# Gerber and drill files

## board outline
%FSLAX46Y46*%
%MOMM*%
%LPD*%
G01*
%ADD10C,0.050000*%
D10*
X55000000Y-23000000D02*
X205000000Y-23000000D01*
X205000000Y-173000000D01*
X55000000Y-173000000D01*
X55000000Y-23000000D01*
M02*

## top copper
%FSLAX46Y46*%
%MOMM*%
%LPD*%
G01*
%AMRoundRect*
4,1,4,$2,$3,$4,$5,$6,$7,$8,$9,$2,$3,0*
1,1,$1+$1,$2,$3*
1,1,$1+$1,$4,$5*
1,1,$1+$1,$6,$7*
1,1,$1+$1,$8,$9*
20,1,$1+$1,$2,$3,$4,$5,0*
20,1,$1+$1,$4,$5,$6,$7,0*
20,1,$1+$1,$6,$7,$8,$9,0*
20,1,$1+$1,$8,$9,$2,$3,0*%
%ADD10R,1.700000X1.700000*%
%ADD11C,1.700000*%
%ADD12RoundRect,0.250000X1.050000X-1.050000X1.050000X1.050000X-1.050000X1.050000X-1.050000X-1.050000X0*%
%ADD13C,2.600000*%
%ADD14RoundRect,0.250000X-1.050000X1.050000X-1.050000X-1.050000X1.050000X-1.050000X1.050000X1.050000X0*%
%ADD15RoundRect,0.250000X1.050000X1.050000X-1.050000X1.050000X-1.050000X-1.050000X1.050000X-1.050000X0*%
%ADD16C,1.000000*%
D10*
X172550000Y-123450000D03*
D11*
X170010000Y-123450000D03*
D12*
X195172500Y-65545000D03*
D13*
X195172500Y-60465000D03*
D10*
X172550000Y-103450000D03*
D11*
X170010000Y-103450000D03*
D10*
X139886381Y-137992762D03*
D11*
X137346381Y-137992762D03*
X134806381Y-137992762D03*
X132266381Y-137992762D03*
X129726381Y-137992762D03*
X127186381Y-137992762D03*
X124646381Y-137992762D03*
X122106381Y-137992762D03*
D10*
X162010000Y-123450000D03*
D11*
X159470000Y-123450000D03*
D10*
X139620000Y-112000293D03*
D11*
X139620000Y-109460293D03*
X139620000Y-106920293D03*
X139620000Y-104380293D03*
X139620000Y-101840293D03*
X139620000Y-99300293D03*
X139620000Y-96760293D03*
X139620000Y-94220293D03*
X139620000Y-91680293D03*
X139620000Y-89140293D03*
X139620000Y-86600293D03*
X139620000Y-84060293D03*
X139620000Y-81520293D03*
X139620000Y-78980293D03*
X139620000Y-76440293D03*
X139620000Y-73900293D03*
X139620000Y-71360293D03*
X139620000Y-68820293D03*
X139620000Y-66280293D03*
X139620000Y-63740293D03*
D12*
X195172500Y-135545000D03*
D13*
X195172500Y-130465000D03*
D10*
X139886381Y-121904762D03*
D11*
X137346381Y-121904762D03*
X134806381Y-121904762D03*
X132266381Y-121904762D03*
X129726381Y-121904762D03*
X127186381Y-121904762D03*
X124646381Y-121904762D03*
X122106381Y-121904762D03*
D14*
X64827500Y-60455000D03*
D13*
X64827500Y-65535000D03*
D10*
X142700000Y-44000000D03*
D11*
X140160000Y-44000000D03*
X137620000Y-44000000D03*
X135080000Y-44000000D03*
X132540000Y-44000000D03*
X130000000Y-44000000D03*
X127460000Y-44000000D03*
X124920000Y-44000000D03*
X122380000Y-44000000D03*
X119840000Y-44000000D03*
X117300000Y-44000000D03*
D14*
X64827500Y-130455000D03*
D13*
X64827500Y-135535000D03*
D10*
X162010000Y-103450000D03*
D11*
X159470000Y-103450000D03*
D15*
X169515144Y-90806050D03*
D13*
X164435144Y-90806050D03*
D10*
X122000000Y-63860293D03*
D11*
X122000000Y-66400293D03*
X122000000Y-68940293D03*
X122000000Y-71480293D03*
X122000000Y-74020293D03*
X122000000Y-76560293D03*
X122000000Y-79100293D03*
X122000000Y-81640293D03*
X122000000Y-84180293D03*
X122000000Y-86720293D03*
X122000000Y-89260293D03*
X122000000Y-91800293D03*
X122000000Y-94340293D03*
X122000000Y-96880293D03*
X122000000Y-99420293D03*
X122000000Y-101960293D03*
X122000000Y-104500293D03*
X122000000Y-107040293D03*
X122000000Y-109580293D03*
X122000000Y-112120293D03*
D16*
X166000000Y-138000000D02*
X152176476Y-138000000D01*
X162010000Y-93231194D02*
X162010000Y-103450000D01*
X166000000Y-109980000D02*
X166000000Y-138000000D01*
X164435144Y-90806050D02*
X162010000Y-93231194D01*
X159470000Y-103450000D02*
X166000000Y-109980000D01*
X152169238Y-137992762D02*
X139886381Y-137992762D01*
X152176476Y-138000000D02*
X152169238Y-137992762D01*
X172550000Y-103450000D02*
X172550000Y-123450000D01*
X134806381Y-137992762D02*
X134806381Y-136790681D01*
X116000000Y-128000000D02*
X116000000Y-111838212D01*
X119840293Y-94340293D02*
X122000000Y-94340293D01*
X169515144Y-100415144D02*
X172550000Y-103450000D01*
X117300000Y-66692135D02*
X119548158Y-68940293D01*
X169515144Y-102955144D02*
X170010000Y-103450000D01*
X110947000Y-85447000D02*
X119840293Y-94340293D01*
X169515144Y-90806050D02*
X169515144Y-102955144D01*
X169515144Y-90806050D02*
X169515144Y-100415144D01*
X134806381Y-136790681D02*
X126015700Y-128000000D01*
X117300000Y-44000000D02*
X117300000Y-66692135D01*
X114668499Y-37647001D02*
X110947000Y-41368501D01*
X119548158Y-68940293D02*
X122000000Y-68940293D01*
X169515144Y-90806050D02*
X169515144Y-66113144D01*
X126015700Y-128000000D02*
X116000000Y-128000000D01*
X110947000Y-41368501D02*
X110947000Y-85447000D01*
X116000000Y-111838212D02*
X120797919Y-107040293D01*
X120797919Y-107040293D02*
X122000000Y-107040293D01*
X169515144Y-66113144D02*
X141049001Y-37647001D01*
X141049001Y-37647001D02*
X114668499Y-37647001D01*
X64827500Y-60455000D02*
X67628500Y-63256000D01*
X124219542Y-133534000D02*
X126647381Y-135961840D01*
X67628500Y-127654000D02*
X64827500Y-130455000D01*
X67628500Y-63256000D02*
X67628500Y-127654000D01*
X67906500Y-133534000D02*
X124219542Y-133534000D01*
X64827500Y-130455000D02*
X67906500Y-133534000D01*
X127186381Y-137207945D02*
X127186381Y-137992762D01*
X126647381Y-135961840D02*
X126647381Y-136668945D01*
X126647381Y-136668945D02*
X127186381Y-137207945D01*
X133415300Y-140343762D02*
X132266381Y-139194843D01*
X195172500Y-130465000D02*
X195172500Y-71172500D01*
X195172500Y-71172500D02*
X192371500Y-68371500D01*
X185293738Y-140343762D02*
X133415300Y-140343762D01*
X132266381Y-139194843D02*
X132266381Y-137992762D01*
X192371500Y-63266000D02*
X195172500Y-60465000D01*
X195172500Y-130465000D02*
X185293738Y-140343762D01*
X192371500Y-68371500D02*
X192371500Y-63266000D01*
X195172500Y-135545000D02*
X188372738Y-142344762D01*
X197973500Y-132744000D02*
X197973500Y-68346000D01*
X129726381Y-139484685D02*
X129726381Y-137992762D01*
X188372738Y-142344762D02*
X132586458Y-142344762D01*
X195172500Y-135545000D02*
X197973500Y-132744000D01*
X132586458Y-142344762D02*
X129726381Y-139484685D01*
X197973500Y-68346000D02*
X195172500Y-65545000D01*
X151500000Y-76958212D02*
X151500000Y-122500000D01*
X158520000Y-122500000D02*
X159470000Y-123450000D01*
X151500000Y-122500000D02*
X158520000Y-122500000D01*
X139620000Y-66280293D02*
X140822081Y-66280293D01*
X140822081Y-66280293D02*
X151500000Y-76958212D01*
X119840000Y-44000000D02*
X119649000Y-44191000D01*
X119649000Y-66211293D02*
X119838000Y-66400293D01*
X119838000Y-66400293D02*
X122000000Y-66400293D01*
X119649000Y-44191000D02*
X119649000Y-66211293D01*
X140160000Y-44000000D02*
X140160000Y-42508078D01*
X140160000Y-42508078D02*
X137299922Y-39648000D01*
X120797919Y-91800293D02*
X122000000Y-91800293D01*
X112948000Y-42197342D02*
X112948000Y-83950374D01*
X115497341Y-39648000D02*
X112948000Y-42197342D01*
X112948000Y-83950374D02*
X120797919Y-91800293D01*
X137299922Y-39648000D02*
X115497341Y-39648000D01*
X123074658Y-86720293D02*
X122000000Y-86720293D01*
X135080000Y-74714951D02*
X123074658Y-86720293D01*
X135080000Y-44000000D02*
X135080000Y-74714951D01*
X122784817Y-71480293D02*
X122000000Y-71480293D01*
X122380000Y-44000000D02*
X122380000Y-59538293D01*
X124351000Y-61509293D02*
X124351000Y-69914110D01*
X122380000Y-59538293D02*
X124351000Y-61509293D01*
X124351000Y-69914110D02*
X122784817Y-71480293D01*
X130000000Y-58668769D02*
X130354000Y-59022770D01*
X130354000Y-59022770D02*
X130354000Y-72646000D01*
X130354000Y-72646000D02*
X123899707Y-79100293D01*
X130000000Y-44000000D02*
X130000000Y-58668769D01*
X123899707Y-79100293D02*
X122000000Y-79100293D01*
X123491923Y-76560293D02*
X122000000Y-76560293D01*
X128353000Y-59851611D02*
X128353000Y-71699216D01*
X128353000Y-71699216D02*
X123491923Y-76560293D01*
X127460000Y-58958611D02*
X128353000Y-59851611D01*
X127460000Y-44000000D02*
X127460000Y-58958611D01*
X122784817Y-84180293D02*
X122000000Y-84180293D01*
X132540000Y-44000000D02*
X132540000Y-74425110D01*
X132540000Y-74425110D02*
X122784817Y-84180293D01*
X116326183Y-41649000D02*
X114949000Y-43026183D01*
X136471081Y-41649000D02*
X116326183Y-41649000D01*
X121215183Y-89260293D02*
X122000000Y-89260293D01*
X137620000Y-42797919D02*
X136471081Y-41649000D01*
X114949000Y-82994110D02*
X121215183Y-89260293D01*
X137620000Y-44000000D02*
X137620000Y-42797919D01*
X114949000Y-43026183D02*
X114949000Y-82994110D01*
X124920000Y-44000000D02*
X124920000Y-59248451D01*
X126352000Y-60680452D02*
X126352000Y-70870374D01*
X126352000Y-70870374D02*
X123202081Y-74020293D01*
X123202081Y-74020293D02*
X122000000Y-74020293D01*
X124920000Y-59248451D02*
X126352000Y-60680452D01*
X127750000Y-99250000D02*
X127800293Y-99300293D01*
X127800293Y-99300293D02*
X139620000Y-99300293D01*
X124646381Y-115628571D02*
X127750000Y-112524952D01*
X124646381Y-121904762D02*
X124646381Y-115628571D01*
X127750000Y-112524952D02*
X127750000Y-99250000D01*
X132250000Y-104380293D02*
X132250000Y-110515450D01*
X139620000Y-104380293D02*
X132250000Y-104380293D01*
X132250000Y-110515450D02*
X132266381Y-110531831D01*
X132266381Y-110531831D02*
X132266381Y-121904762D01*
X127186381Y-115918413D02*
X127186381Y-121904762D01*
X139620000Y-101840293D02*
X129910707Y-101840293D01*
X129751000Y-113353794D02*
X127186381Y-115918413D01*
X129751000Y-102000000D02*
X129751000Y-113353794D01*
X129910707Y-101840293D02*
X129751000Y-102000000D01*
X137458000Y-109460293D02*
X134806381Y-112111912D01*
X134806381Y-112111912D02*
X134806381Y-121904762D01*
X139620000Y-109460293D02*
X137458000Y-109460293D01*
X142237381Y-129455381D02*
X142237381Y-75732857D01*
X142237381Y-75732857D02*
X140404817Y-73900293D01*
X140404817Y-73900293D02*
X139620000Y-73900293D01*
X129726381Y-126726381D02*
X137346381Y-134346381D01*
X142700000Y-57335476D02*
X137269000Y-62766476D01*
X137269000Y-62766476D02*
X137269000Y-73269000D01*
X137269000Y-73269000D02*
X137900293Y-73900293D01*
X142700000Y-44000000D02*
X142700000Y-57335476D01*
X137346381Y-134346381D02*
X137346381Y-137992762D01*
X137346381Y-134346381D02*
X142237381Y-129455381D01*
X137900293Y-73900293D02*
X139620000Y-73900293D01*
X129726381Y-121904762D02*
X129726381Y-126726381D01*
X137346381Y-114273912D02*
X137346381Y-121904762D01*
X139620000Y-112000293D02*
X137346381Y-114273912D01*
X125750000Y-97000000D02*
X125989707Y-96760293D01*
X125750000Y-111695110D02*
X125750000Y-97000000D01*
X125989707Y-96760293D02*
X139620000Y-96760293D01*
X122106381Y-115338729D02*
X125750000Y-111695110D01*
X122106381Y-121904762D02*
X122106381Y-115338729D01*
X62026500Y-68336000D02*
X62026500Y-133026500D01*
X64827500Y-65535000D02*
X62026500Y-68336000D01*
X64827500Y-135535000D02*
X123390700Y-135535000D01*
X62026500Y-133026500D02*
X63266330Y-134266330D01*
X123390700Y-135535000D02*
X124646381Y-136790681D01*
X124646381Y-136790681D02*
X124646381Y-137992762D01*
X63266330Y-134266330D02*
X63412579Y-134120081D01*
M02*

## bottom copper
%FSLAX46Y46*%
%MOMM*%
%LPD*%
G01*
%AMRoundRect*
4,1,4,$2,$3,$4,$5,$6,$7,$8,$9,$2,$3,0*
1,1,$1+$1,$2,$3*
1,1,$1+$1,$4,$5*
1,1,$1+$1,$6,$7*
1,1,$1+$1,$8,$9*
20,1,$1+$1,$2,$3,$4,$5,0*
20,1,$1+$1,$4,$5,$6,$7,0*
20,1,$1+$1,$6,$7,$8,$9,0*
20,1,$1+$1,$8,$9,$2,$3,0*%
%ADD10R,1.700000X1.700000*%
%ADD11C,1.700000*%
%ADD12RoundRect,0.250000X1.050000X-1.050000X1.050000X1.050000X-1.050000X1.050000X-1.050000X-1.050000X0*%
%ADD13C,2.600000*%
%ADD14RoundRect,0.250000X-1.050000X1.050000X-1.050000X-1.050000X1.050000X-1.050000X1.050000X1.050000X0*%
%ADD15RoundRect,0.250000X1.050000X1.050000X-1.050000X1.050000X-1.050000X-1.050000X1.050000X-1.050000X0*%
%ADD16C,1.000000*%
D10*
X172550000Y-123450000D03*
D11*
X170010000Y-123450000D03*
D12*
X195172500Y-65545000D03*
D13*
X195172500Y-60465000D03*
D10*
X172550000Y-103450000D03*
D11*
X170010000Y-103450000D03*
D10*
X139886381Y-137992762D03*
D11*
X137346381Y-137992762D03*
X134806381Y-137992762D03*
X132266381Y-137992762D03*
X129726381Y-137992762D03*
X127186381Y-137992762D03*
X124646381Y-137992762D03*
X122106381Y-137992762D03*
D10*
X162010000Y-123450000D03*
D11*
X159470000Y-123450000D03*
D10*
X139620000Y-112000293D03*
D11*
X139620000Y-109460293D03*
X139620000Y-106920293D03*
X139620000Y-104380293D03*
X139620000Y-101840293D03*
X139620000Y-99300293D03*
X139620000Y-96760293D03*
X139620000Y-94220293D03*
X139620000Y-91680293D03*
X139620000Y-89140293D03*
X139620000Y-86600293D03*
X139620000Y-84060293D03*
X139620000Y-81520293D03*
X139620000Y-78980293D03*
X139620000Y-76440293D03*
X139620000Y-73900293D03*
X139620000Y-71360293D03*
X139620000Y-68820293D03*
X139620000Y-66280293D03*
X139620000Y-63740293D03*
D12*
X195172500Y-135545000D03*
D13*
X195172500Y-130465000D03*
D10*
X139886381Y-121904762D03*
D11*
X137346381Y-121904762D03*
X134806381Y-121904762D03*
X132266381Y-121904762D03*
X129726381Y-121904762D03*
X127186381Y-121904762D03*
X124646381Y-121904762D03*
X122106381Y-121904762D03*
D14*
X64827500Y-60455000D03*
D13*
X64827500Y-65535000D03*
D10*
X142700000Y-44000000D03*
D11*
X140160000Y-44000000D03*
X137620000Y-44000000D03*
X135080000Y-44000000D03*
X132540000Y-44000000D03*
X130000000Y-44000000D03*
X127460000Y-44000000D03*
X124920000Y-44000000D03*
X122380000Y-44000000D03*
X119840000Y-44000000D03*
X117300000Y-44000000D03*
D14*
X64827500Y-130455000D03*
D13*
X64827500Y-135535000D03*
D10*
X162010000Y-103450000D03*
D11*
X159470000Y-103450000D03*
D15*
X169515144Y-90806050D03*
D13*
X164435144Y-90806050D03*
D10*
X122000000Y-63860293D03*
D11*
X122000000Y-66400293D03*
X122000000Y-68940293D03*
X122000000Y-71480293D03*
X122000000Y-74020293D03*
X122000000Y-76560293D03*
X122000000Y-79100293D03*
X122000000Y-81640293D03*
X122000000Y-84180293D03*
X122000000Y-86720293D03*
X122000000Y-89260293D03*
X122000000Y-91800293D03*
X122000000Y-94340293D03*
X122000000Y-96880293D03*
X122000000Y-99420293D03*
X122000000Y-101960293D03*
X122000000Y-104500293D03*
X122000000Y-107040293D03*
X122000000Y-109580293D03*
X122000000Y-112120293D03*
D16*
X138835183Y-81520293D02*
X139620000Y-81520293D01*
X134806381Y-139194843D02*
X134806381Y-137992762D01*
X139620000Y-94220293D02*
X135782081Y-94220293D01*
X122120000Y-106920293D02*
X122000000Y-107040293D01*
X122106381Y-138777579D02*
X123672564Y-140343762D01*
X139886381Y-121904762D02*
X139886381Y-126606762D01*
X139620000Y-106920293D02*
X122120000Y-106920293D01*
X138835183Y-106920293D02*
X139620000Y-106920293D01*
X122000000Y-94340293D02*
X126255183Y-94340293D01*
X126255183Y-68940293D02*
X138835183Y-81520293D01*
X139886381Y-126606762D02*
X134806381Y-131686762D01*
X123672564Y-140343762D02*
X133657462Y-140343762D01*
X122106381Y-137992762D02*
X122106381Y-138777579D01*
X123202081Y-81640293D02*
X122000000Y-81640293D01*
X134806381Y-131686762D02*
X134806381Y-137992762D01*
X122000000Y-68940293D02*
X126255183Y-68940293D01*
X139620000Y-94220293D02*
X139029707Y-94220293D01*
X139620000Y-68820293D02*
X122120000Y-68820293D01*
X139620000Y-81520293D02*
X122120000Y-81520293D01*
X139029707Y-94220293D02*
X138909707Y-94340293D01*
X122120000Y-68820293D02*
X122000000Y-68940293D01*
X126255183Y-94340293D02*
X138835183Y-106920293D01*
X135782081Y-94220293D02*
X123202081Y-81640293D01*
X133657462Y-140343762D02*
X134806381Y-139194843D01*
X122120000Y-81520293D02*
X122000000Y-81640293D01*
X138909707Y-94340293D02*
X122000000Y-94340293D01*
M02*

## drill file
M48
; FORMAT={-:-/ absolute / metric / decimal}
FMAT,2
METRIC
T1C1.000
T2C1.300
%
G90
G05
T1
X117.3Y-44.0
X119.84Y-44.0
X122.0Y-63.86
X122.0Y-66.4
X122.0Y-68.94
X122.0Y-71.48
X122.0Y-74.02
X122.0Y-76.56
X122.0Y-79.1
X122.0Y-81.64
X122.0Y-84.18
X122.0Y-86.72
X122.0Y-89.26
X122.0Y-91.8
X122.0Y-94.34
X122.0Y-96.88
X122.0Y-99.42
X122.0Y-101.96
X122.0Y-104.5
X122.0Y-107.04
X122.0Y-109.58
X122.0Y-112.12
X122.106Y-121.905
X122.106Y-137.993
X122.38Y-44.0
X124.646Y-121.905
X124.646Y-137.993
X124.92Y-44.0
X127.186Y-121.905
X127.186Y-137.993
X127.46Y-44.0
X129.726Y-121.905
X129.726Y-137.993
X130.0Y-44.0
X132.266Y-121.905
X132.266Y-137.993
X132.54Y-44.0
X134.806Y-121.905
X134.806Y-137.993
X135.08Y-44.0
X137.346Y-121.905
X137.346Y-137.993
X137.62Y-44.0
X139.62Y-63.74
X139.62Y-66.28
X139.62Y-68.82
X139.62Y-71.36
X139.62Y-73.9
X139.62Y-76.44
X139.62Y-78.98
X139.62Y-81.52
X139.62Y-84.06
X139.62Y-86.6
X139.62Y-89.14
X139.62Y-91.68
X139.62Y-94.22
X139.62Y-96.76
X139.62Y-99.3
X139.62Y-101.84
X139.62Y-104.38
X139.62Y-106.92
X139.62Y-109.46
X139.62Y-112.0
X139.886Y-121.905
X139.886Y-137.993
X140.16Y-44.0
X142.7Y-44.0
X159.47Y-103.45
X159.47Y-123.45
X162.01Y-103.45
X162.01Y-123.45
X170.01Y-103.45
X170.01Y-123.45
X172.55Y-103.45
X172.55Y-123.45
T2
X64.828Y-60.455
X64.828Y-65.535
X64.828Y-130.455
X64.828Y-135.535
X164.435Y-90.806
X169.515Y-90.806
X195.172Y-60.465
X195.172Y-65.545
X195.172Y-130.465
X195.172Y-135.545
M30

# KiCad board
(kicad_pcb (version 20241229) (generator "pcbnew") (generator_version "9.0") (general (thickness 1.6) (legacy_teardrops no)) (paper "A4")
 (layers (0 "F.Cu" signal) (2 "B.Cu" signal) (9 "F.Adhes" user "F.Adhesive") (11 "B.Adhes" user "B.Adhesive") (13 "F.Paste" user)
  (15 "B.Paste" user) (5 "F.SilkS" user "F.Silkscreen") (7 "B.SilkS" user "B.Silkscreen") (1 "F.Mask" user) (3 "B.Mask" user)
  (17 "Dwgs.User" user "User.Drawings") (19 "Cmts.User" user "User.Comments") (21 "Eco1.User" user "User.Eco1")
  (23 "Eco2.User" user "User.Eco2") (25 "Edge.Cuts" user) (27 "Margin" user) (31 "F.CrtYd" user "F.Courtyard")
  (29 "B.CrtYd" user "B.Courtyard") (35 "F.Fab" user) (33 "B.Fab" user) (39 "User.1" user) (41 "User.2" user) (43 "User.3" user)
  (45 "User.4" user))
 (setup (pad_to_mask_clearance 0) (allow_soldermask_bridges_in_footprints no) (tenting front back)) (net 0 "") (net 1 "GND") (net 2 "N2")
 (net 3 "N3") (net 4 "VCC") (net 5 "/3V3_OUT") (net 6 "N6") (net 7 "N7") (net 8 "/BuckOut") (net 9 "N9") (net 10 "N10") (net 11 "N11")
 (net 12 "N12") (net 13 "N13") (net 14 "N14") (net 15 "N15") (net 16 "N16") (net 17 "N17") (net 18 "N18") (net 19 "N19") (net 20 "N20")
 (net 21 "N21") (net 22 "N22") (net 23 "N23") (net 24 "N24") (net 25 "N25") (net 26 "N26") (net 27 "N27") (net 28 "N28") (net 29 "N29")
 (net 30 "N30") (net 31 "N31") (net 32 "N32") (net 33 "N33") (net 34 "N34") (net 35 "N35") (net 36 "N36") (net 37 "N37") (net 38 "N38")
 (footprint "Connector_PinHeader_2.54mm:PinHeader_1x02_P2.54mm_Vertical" (layer "F.Cu") (at 172.55 123.45 -90)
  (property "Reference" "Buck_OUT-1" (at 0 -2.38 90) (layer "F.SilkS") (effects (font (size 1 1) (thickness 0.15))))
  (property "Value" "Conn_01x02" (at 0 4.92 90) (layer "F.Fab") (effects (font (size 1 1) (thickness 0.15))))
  (pad "1" thru_hole rect (at 0 0 270) (size 1.7 1.7) (drill 1) (layers "*.Cu" "*.Mask") (remove_unused_layers no) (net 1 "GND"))
  (pad "2" thru_hole circle (at 0 2.54 270) (size 1.7 1.7) (drill 1) (layers "*.Cu" "*.Mask") (remove_unused_layers no) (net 1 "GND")))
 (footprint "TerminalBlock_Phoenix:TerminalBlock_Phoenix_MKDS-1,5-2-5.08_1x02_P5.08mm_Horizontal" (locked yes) (layer "F.Cu")
  (at 195.1725 65.545 90)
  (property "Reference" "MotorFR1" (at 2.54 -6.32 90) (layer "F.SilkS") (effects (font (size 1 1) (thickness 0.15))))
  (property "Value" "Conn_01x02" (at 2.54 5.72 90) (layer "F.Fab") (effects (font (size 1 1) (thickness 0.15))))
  (pad "1" thru_hole roundrect (at 0 0 90) (size 2.6 2.6) (drill 1.3) (layers "*.Cu" "*.Mask") (remove_unused_layers no)
   (roundrect_rratio 0.096154) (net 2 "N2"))
  (pad "2" thru_hole circle (at 5.08 0 90) (size 2.6 2.6) (drill 1.3) (layers "*.Cu" "*.Mask") (remove_unused_layers no) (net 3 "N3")))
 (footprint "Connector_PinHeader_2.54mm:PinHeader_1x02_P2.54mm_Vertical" (layer "F.Cu") (at 172.55 103.45 -90)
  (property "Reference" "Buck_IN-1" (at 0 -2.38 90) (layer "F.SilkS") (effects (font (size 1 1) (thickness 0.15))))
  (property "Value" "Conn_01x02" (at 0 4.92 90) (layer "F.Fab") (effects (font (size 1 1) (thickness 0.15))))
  (pad "1" thru_hole rect (at 0 0 270) (size 1.7 1.7) (drill 1) (layers "*.Cu" "*.Mask") (remove_unused_layers no) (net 1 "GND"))
  (pad "2" thru_hole circle (at 0 2.54 270) (size 1.7 1.7) (drill 1) (layers "*.Cu" "*.Mask") (remove_unused_layers no) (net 1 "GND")))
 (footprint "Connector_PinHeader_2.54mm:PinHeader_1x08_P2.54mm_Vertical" (layer "F.Cu") (at 139.886381 137.992762 -90)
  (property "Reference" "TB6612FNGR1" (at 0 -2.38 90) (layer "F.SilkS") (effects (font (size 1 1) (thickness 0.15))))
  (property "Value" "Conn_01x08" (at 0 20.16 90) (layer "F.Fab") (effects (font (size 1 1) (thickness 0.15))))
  (pad "1" thru_hole rect (at 0 0 270) (size 1.7 1.7) (drill 1) (layers "*.Cu" "*.Mask") (remove_unused_layers no) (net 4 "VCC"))
  (pad "2" thru_hole circle (at 0 2.54 270) (size 1.7 1.7) (drill 1) (layers "*.Cu" "*.Mask") (remove_unused_layers no) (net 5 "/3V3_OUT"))
  (pad "3" thru_hole circle (at 0 5.08 270) (size 1.7 1.7) (drill 1) (layers "*.Cu" "*.Mask") (remove_unused_layers no) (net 1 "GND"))
  (pad "4" thru_hole circle (at 0 7.62 270) (size 1.7 1.7) (drill 1) (layers "*.Cu" "*.Mask") (remove_unused_layers no) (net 3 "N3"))
  (pad "5" thru_hole circle (at 0 10.16 270) (size 1.7 1.7) (drill 1) (layers "*.Cu" "*.Mask") (remove_unused_layers no) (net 2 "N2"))
  (pad "6" thru_hole circle (at 0 12.7 270) (size 1.7 1.7) (drill 1) (layers "*.Cu" "*.Mask") (remove_unused_layers no) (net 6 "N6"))
  (pad "7" thru_hole circle (at 0 15.24 270) (size 1.7 1.7) (drill 1) (layers "*.Cu" "*.Mask") (remove_unused_layers no) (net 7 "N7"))
  (pad "8" thru_hole circle (at 0 17.78 270) (size 1.7 1.7) (drill 1) (layers "*.Cu" "*.Mask") (remove_unused_layers no) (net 1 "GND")))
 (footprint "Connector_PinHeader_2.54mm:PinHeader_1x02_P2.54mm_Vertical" (layer "F.Cu") (at 162.01 123.45 -90)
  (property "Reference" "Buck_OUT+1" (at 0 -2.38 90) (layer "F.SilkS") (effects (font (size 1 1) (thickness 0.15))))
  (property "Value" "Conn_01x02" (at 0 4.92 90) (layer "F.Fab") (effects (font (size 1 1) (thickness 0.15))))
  (pad "1" thru_hole rect (at 0 0 270) (size 1.7 1.7) (drill 1) (layers "*.Cu" "*.Mask") (remove_unused_layers no) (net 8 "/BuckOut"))
  (pad "2" thru_hole circle (at 0 2.54 270) (size 1.7 1.7) (drill 1) (layers "*.Cu" "*.Mask") (remove_unused_layers no) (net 8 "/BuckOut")))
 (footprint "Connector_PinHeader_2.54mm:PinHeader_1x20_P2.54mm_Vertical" (layer "F.Cu") (at 139.62 112.000293 180)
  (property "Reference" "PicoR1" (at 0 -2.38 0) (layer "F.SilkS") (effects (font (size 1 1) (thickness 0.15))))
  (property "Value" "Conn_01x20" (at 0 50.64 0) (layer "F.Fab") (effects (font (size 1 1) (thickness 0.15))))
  (pad "1" thru_hole rect (at 0 0 180) (size 1.7 1.7) (drill 1) (layers "*.Cu" "*.Mask") (remove_unused_layers no) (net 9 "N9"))
  (pad "2" thru_hole circle (at 0 2.54 180) (size 1.7 1.7) (drill 1) (layers "*.Cu" "*.Mask") (remove_unused_layers no) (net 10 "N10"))
  (pad "3" thru_hole circle (at 0 5.08 180) (size 1.7 1.7) (drill 1) (layers "*.Cu" "*.Mask") (remove_unused_layers no) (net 1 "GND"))
  (pad "4" thru_hole circle (at 0 7.62 180) (size 1.7 1.7) (drill 1) (layers "*.Cu" "*.Mask") (remove_unused_layers no) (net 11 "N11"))
  (pad "5" thru_hole circle (at 0 10.16 180) (size 1.7 1.7) (drill 1) (layers "*.Cu" "*.Mask") (remove_unused_layers no) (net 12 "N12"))
  (pad "6" thru_hole circle (at 0 12.7 180) (size 1.7 1.7) (drill 1) (layers "*.Cu" "*.Mask") (remove_unused_layers no) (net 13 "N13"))
  (pad "7" thru_hole circle (at 0 15.24 180) (size 1.7 1.7) (drill 1) (layers "*.Cu" "*.Mask") (remove_unused_layers no) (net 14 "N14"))
  (pad "8" thru_hole circle (at 0 17.78 180) (size 1.7 1.7) (drill 1) (layers "*.Cu" "*.Mask") (remove_unused_layers no) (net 1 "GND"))
  (pad "9" thru_hole circle (at 0 20.32 180) (size 1.7 1.7) (drill 1) (layers "*.Cu" "*.Mask") (remove_unused_layers no) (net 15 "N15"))
  (pad "10" thru_hole circle (at 0 22.86 180) (size 1.7 1.7) (drill 1) (layers "*.Cu" "*.Mask") (remove_unused_layers no) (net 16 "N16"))
  (pad "11" thru_hole circle (at 0 25.4 180) (size 1.7 1.7) (drill 1) (layers "*.Cu" "*.Mask") (remove_unused_layers no) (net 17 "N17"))
  (pad "12" thru_hole circle (at 0 27.94 180) (size 1.7 1.7) (drill 1) (layers "*.Cu" "*.Mask") (remove_unused_layers no) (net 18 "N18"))
  (pad "13" thru_hole circle (at 0 30.48 180) (size 1.7 1.7) (drill 1) (layers "*.Cu" "*.Mask") (remove_unused_layers no) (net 1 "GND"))
  (pad "14" thru_hole circle (at 0 33.02 180) (size 1.7 1.7) (drill 1) (layers "*.Cu" "*.Mask") (remove_unused_layers no) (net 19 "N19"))
  (pad "15" thru_hole circle (at 0 35.56 180) (size 1.7 1.7) (drill 1) (layers "*.Cu" "*.Mask") (remove_unused_layers no) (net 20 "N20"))
  (pad "16" thru_hole circle (at 0 38.1 180) (size 1.7 1.7) (drill 1) (layers "*.Cu" "*.Mask") (remove_unused_layers no) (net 5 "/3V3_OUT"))
  (pad "17" thru_hole circle (at 0 40.64 180) (size 1.7 1.7) (drill 1) (layers "*.Cu" "*.Mask") (remove_unused_layers no) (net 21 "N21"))
  (pad "18" thru_hole circle (at 0 43.18 180) (size 1.7 1.7) (drill 1) (layers "*.Cu" "*.Mask") (remove_unused_layers no) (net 1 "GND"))
  (pad "19" thru_hole circle (at 0 45.72 180) (size 1.7 1.7) (drill 1) (layers "*.Cu" "*.Mask") (remove_unused_layers no) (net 8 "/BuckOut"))
  (pad "20" thru_hole circle (at 0 48.26 180) (size 1.7 1.7) (drill 1) (layers "*.Cu" "*.Mask") (remove_unused_layers no) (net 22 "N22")))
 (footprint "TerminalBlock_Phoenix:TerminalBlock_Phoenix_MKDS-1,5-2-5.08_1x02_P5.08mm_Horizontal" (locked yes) (layer "F.Cu")
  (at 195.1725 135.545 90)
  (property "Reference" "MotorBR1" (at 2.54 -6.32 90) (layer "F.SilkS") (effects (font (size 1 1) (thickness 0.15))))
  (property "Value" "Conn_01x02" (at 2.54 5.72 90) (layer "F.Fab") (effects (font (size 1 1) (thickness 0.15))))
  (pad "1" thru_hole roundrect (at 0 0 90) (size 2.6 2.6) (drill 1.3) (layers "*.Cu" "*.Mask") (remove_unused_layers no)
   (roundrect_rratio 0.096154) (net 2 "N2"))
  (pad "2" thru_hole circle (at 5.08 0 90) (size 2.6 2.6) (drill 1.3) (layers "*.Cu" "*.Mask") (remove_unused_layers no) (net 3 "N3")))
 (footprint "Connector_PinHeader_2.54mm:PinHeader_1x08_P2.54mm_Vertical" (layer "F.Cu") (at 139.886381 121.904762 -90)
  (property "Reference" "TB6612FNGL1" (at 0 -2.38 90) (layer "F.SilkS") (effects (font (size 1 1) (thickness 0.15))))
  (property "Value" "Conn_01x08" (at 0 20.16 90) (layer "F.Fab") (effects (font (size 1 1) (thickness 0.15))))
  (pad "1" thru_hole rect (at 0 0 270) (size 1.7 1.7) (drill 1) (layers "*.Cu" "*.Mask") (remove_unused_layers no) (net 1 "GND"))
  (pad "2" thru_hole circle (at 0 2.54 270) (size 1.7 1.7) (drill 1) (layers "*.Cu" "*.Mask") (remove_unused_layers no) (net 9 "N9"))
  (pad "3" thru_hole circle (at 0 5.08 270) (size 1.7 1.7) (drill 1) (layers "*.Cu" "*.Mask") (remove_unused_layers no) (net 10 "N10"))
  (pad "4" thru_hole circle (at 0 7.62 270) (size 1.7 1.7) (drill 1) (layers "*.Cu" "*.Mask") (remove_unused_layers no) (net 11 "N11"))
  (pad "5" thru_hole circle (at 0 10.16 270) (size 1.7 1.7) (drill 1) (layers "*.Cu" "*.Mask") (remove_unused_layers no) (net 5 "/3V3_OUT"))
  (pad "6" thru_hole circle (at 0 12.7 270) (size 1.7 1.7) (drill 1) (layers "*.Cu" "*.Mask") (remove_unused_layers no) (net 12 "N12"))
  (pad "7" thru_hole circle (at 0 15.24 270) (size 1.7 1.7) (drill 1) (layers "*.Cu" "*.Mask") (remove_unused_layers no) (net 13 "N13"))
  (pad "8" thru_hole circle (at 0 17.78 270) (size 1.7 1.7) (drill 1) (layers "*.Cu" "*.Mask") (remove_unused_layers no) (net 14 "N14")))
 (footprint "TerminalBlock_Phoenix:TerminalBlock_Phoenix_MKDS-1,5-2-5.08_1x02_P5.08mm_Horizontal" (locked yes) (layer "F.Cu")
  (at 64.8275 60.455 -90)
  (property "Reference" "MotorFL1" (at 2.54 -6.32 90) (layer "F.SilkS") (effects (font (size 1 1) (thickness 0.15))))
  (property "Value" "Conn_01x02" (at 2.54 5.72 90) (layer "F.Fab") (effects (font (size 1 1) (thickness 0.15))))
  (pad "1" thru_hole roundrect (at 0 0 270) (size 2.6 2.6) (drill 1.3) (layers "*.Cu" "*.Mask") (remove_unused_layers no)
   (roundrect_rratio 0.096154) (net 6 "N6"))
  (pad "2" thru_hole circle (at 5.08 0 270) (size 2.6 2.6) (drill 1.3) (layers "*.Cu" "*.Mask") (remove_unused_layers no) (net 7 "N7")))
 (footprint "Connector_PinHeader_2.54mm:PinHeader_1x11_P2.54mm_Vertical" (layer "F.Cu") (at 142.7 44 -90)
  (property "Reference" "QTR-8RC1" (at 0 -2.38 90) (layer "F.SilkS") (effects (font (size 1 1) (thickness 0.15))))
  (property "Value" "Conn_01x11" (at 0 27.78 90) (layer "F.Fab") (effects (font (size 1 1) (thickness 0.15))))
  (pad "1" thru_hole rect (at 0 0 270) (size 1.7 1.7) (drill 1) (layers "*.Cu" "*.Mask") (remove_unused_layers no) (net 5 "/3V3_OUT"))
  (pad "2" thru_hole circle (at 0 2.54 270) (size 1.7 1.7) (drill 1) (layers "*.Cu" "*.Mask") (remove_unused_layers no) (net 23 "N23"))
  (pad "3" thru_hole circle (at 0 5.08 270) (size 1.7 1.7) (drill 1) (layers "*.Cu" "*.Mask") (remove_unused_layers no) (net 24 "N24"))
  (pad "4" thru_hole circle (at 0 7.62 270) (size 1.7 1.7) (drill 1) (layers "*.Cu" "*.Mask") (remove_unused_layers no) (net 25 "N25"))
  (pad "5" thru_hole circle (at 0 10.16 270) (size 1.7 1.7) (drill 1) (layers "*.Cu" "*.Mask") (remove_unused_layers no) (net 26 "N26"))
  (pad "6" thru_hole circle (at 0 12.7 270) (size 1.7 1.7) (drill 1) (layers "*.Cu" "*.Mask") (remove_unused_layers no) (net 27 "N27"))
  (pad "7" thru_hole circle (at 0 15.24 270) (size 1.7 1.7) (drill 1) (layers "*.Cu" "*.Mask") (remove_unused_layers no) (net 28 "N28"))
  (pad "8" thru_hole circle (at 0 17.78 270) (size 1.7 1.7) (drill 1) (layers "*.Cu" "*.Mask") (remove_unused_layers no) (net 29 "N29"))
  (pad "9" thru_hole circle (at 0 20.32 270) (size 1.7 1.7) (drill 1) (layers "*.Cu" "*.Mask") (remove_unused_layers no) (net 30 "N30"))
  (pad "10" thru_hole circle (at 0 22.86 270) (size 1.7 1.7) (drill 1) (layers "*.Cu" "*.Mask") (remove_unused_layers no) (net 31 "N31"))
  (pad "11" thru_hole circle (at 0 25.4 270) (size 1.7 1.7) (drill 1) (layers "*.Cu" "*.Mask") (remove_unused_layers no) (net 1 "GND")))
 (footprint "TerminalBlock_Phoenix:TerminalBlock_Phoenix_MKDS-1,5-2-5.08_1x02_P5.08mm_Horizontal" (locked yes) (layer "F.Cu")
  (at 64.8275 130.455 -90)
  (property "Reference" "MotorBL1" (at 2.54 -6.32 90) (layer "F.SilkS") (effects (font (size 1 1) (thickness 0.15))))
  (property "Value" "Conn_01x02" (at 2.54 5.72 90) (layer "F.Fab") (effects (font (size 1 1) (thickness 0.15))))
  (pad "1" thru_hole roundrect (at 0 0 270) (size 2.6 2.6) (drill 1.3) (layers "*.Cu" "*.Mask") (remove_unused_layers no)
   (roundrect_rratio 0.096154) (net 6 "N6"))
  (pad "2" thru_hole circle (at 5.08 0 270) (size 2.6 2.6) (drill 1.3) (layers "*.Cu" "*.Mask") (remove_unused_layers no) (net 7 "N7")))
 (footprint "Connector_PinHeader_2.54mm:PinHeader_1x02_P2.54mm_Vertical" (layer "F.Cu") (at 162.01 103.45 -90)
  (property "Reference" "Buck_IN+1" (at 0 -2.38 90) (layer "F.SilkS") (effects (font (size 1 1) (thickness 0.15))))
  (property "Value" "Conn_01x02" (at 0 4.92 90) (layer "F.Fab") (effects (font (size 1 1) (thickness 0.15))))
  (pad "1" thru_hole rect (at 0 0 270) (size 1.7 1.7) (drill 1) (layers "*.Cu" "*.Mask") (remove_unused_layers no) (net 4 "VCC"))
  (pad "2" thru_hole circle (at 0 2.54 270) (size 1.7 1.7) (drill 1) (layers "*.Cu" "*.Mask") (remove_unused_layers no) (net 4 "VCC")))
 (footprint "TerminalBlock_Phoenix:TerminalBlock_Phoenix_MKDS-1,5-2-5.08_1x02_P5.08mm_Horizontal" (layer "F.Cu")
  (at 169.515144 90.80605 180)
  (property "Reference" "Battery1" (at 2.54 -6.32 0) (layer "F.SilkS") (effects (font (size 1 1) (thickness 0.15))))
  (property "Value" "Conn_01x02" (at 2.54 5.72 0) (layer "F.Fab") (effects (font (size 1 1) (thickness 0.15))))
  (pad "1" thru_hole roundrect (at 0 0 180) (size 2.6 2.6) (drill 1.3) (layers "*.Cu" "*.Mask") (remove_unused_layers no)
   (roundrect_rratio 0.096154) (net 1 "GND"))
  (pad "2" thru_hole circle (at 5.08 0 180) (size 2.6 2.6) (drill 1.3) (layers "*.Cu" "*.Mask") (remove_unused_layers no) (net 4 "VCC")))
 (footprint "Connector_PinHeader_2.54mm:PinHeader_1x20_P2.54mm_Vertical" (layer "F.Cu") (at 122 63.860293)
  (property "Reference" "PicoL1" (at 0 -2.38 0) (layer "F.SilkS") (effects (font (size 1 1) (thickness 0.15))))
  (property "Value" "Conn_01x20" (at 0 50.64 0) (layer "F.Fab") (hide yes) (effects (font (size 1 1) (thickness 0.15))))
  (pad "1" thru_hole rect (at 0 0) (size 1.7 1.7) (drill 1) (layers "*.Cu" "*.Mask") (remove_unused_layers no) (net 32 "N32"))
  (pad "2" thru_hole circle (at 0 2.54) (size 1.7 1.7) (drill 1) (layers "*.Cu" "*.Mask") (remove_unused_layers no) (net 31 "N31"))
  (pad "3" thru_hole circle (at 0 5.08) (size 1.7 1.7) (drill 1) (layers "*.Cu" "*.Mask") (remove_unused_layers no) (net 1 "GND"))
  (pad "4" thru_hole circle (at 0 7.62) (size 1.7 1.7) (drill 1) (layers "*.Cu" "*.Mask") (remove_unused_layers no) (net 30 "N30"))
  (pad "5" thru_hole circle (at 0 10.16) (size 1.7 1.7) (drill 1) (layers "*.Cu" "*.Mask") (remove_unused_layers no) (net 29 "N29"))
  (pad "6" thru_hole circle (at 0 12.7) (size 1.7 1.7) (drill 1) (layers "*.Cu" "*.Mask") (remove_unused_layers no) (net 28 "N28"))
  (pad "7" thru_hole circle (at 0 15.24) (size 1.7 1.7) (drill 1) (layers "*.Cu" "*.Mask") (remove_unused_layers no) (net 27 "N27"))
  (pad "8" thru_hole circle (at 0 17.78) (size 1.7 1.7) (drill 1) (layers "*.Cu" "*.Mask") (remove_unused_layers no) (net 1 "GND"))
  (pad "9" thru_hole circle (at 0 20.32) (size 1.7 1.7) (drill 1) (layers "*.Cu" "*.Mask") (remove_unused_layers no) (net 26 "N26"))
  (pad "10" thru_hole circle (at 0 22.86) (size 1.7 1.7) (drill 1) (layers "*.Cu" "*.Mask") (remove_unused_layers no) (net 25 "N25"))
  (pad "11" thru_hole circle (at 0 25.4) (size 1.7 1.7) (drill 1) (layers "*.Cu" "*.Mask") (remove_unused_layers no) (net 24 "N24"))
  (pad "12" thru_hole circle (at 0 27.94) (size 1.7 1.7) (drill 1) (layers "*.Cu" "*.Mask") (remove_unused_layers no) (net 23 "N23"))
  (pad "13" thru_hole circle (at 0 30.48) (size 1.7 1.7) (drill 1) (layers "*.Cu" "*.Mask") (remove_unused_layers no) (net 1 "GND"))
  (pad "14" thru_hole circle (at 0 33.02) (size 1.7 1.7) (drill 1) (layers "*.Cu" "*.Mask") (remove_unused_layers no) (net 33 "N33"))
  (pad "15" thru_hole circle (at 0 35.56) (size 1.7 1.7) (drill 1) (layers "*.Cu" "*.Mask") (remove_unused_layers no) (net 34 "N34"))
  (pad "16" thru_hole circle (at 0 38.1) (size 1.7 1.7) (drill 1) (layers "*.Cu" "*.Mask") (remove_unused_layers no) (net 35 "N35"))
  (pad "17" thru_hole circle (at 0 40.64) (size 1.7 1.7) (drill 1) (layers "*.Cu" "*.Mask") (remove_unused_layers no) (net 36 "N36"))
  (pad "18" thru_hole circle (at 0 43.18) (size 1.7 1.7) (drill 1) (layers "*.Cu" "*.Mask") (remove_unused_layers no) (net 1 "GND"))
  (pad "19" thru_hole circle (at 0 45.72) (size 1.7 1.7) (drill 1) (layers "*.Cu" "*.Mask") (remove_unused_layers no) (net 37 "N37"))
  (pad "20" thru_hole circle (at 0 48.26) (size 1.7 1.7) (drill 1) (layers "*.Cu" "*.Mask") (remove_unused_layers no) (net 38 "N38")))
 (gr_rect (start 55 23) (end 205 173) (stroke (width 0.05) (type default)) (fill no) (layer "Edge.Cuts"))
 (segment (start 166 138) (end 152.176476 138) (width 1) (layer "F.Cu") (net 4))
 (segment (start 162.01 93.231194) (end 162.01 103.45) (width 1) (layer "F.Cu") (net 4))
 (segment (start 166 109.98) (end 166 138) (width 1) (layer "F.Cu") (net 4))
 (segment (start 164.435144 90.80605) (end 162.01 93.231194) (width 1) (layer "F.Cu") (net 4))
 (segment (start 159.47 103.45) (end 166 109.98) (width 1) (layer "F.Cu") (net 4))
 (segment (start 152.169238 137.992762) (end 139.886381 137.992762) (width 1) (layer "F.Cu") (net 4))
 (segment (start 152.176476 138) (end 152.169238 137.992762) (width 1) (layer "F.Cu") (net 4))
 (segment (start 172.55 103.45) (end 172.55 123.45) (width 1) (layer "F.Cu") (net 1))
 (segment (start 134.806381 137.992762) (end 134.806381 136.790681) (width 1) (layer "F.Cu") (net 1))
 (segment (start 116 128) (end 116 111.838212) (width 1) (layer "F.Cu") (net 1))
 (segment (start 119.840293 94.340293) (end 122 94.340293) (width 1) (layer "F.Cu") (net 1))
 (segment (start 169.515144 100.415144) (end 172.55 103.45) (width 1) (layer "F.Cu") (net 1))
 (segment (start 117.3 66.692135) (end 119.548158 68.940293) (width 1) (layer "F.Cu") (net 1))
 (segment (start 169.515144 102.955144) (end 170.01 103.45) (width 1) (layer "F.Cu") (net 1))
 (segment (start 110.947 85.447) (end 119.840293 94.340293) (width 1) (layer "F.Cu") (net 1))
 (segment (start 169.515144 90.80605) (end 169.515144 102.955144) (width 1) (layer "F.Cu") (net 1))
 (segment (start 169.515144 90.80605) (end 169.515144 100.415144) (width 1) (layer "F.Cu") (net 1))
 (segment (start 134.806381 136.790681) (end 126.0157 128) (width 1) (layer "F.Cu") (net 1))
 (segment (start 117.3 44) (end 117.3 66.692135) (width 1) (layer "F.Cu") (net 1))
 (segment (start 114.668499 37.647001) (end 110.947 41.368501) (width 1) (layer "F.Cu") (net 1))
 (segment (start 119.548158 68.940293) (end 122 68.940293) (width 1) (layer "F.Cu") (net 1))
 (segment (start 169.515144 90.80605) (end 169.515144 66.113144) (width 1) (layer "F.Cu") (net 1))
 (segment (start 126.0157 128) (end 116 128) (width 1) (layer "F.Cu") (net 1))
 (segment (start 110.947 41.368501) (end 110.947 85.447) (width 1) (layer "F.Cu") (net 1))
 (segment (start 116 111.838212) (end 120.797919 107.040293) (width 1) (layer "F.Cu") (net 1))
 (segment (start 120.797919 107.040293) (end 122 107.040293) (width 1) (layer "F.Cu") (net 1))
 (segment (start 169.515144 66.113144) (end 141.049001 37.647001) (width 1) (layer "F.Cu") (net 1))
 (segment (start 141.049001 37.647001) (end 114.668499 37.647001) (width 1) (layer "F.Cu") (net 1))
 (segment (start 138.835183 81.520293) (end 139.62 81.520293) (width 1) (layer "B.Cu") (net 1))
 (segment (start 134.806381 139.194843) (end 134.806381 137.992762) (width 1) (layer "B.Cu") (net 1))
 (segment (start 139.62 94.220293) (end 135.782081 94.220293) (width 1) (layer "B.Cu") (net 1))
 (segment (start 122.12 106.920293) (end 122 107.040293) (width 1) (layer "B.Cu") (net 1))
 (segment (start 122.106381 138.777579) (end 123.672564 140.343762) (width 1) (layer "B.Cu") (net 1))
 (segment (start 139.886381 121.904762) (end 139.886381 126.606762) (width 1) (layer "B.Cu") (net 1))
 (segment (start 139.62 106.920293) (end 122.12 106.920293) (width 1) (layer "B.Cu") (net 1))
 (segment (start 138.835183 106.920293) (end 139.62 106.920293) (width 1) (layer "B.Cu") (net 1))
 (segment (start 122 94.340293) (end 126.255183 94.340293) (width 1) (layer "B.Cu") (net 1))
 (segment (start 126.255183 68.940293) (end 138.835183 81.520293) (width 1) (layer "B.Cu") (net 1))
 (segment (start 139.886381 126.606762) (end 134.806381 131.686762) (width 1) (layer "B.Cu") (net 1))
 (segment (start 123.672564 140.343762) (end 133.657462 140.343762) (width 1) (layer "B.Cu") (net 1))
 (segment (start 122.106381 137.992762) (end 122.106381 138.777579) (width 1) (layer "B.Cu") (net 1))
 (segment (start 123.202081 81.640293) (end 122 81.640293) (width 1) (layer "B.Cu") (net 1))
 (segment (start 134.806381 131.686762) (end 134.806381 137.992762) (width 1) (layer "B.Cu") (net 1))
 (segment (start 122 68.940293) (end 126.255183 68.940293) (width 1) (layer "B.Cu") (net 1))
 (segment (start 139.62 94.220293) (end 139.029707 94.220293) (width 1) (layer "B.Cu") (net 1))
 (segment (start 139.62 68.820293) (end 122.12 68.820293) (width 1) (layer "B.Cu") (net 1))
 (segment (start 139.62 81.520293) (end 122.12 81.520293) (width 1) (layer "B.Cu") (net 1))
 (segment (start 139.029707 94.220293) (end 138.909707 94.340293) (width 1) (layer "B.Cu") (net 1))
 (segment (start 122.12 68.820293) (end 122 68.940293) (width 1) (layer "B.Cu") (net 1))
 (segment (start 126.255183 94.340293) (end 138.835183 106.920293) (width 1) (layer "B.Cu") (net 1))
 (segment (start 135.782081 94.220293) (end 123.202081 81.640293) (width 1) (layer "B.Cu") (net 1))
 (segment (start 133.657462 140.343762) (end 134.806381 139.194843) (width 1) (layer "B.Cu") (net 1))
 (segment (start 122.12 81.520293) (end 122 81.640293) (width 1) (layer "B.Cu") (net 1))
 (segment (start 138.909707 94.340293) (end 122 94.340293) (width 1) (layer "B.Cu") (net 1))
 (segment (start 64.8275 60.455) (end 67.6285 63.256) (width 1) (layer "F.Cu") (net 6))
 (segment (start 124.219542 133.534) (end 126.647381 135.96184) (width 1) (layer "F.Cu") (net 6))
 (segment (start 67.6285 127.654) (end 64.8275 130.455) (width 1) (layer "F.Cu") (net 6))
 (segment (start 67.6285 63.256) (end 67.6285 127.654) (width 1) (layer "F.Cu") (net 6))
 (segment (start 67.9065 133.534) (end 124.219542 133.534) (width 1) (layer "F.Cu") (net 6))
 (segment (start 64.8275 130.455) (end 67.9065 133.534) (width 1) (layer "F.Cu") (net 6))
 (segment (start 127.186381 137.207945) (end 127.186381 137.992762) (width 1) (layer "F.Cu") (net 6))
 (segment (start 126.647381 135.96184) (end 126.647381 136.668945) (width 1) (layer "F.Cu") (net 6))
 (segment (start 126.647381 136.668945) (end 127.186381 137.207945) (width 1) (layer "F.Cu") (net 6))
 (segment (start 133.4153 140.343762) (end 132.266381 139.194843) (width 1) (layer "F.Cu") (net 3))
 (segment (start 195.1725 130.465) (end 195.1725 71.1725) (width 1) (layer "F.Cu") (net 3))
 (segment (start 195.1725 71.1725) (end 192.3715 68.3715) (width 1) (layer "F.Cu") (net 3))
 (segment (start 185.293738 140.343762) (end 133.4153 140.343762) (width 1) (layer "F.Cu") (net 3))
 (segment (start 132.266381 139.194843) (end 132.266381 137.992762) (width 1) (layer "F.Cu") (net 3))
 (segment (start 192.3715 63.266) (end 195.1725 60.465) (width 1) (layer "F.Cu") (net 3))
 (segment (start 195.1725 130.465) (end 185.293738 140.343762) (width 1) (layer "F.Cu") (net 3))
 (segment (start 192.3715 68.3715) (end 192.3715 63.266) (width 1) (layer "F.Cu") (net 3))
 (segment (start 195.1725 135.545) (end 188.372738 142.344762) (width 1) (layer "F.Cu") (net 2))
 (segment (start 197.9735 132.744) (end 197.9735 68.346) (width 1) (layer "F.Cu") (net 2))
 (segment (start 129.726381 139.484685) (end 129.726381 137.992762) (width 1) (layer "F.Cu") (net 2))
 (segment (start 188.372738 142.344762) (end 132.586458 142.344762) (width 1) (layer "F.Cu") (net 2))
 (segment (start 195.1725 135.545) (end 197.9735 132.744) (width 1) (layer "F.Cu") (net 2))
 (segment (start 132.586458 142.344762) (end 129.726381 139.484685) (width 1) (layer "F.Cu") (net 2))
 (segment (start 197.9735 68.346) (end 195.1725 65.545) (width 1) (layer "F.Cu") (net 2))
 (segment (start 151.5 76.958212) (end 151.5 122.5) (width 1) (layer "F.Cu") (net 8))
 (segment (start 158.52 122.5) (end 159.47 123.45) (width 1) (layer "F.Cu") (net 8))
 (segment (start 151.5 122.5) (end 158.52 122.5) (width 1) (layer "F.Cu") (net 8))
 (segment (start 139.62 66.280293) (end 140.822081 66.280293) (width 1) (layer "F.Cu") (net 8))
 (segment (start 140.822081 66.280293) (end 151.5 76.958212) (width 1) (layer "F.Cu") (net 8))
 (segment (start 119.84 44) (end 119.649 44.191) (width 1) (layer "F.Cu") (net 31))
 (segment (start 119.649 66.211293) (end 119.838 66.400293) (width 1) (layer "F.Cu") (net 31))
 (segment (start 119.838 66.400293) (end 122 66.400293) (width 1) (layer "F.Cu") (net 31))
 (segment (start 119.649 44.191) (end 119.649 66.211293) (width 1) (layer "F.Cu") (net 31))
 (segment (start 140.16 44) (end 140.16 42.508078) (width 1) (layer "F.Cu") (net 23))
 (segment (start 140.16 42.508078) (end 137.299922 39.648) (width 1) (layer "F.Cu") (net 23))
 (segment (start 120.797919 91.800293) (end 122 91.800293) (width 1) (layer "F.Cu") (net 23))
 (segment (start 112.948 42.197342) (end 112.948 83.950374) (width 1) (layer "F.Cu") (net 23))
 (segment (start 115.497341 39.648) (end 112.948 42.197342) (width 1) (layer "F.Cu") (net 23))
 (segment (start 112.948 83.950374) (end 120.797919 91.800293) (width 1) (layer "F.Cu") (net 23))
 (segment (start 137.299922 39.648) (end 115.497341 39.648) (width 1) (layer "F.Cu") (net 23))
 (segment (start 123.074658 86.720293) (end 122 86.720293) (width 1) (layer "F.Cu") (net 25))
 (segment (start 135.08 74.714951) (end 123.074658 86.720293) (width 1) (layer "F.Cu") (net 25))
 (segment (start 135.08 44) (end 135.08 74.714951) (width 1) (layer "F.Cu") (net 25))
 (segment (start 122.784817 71.480293) (end 122 71.480293) (width 1) (layer "F.Cu") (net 30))
 (segment (start 122.38 44) (end 122.38 59.538293) (width 1) (layer "F.Cu") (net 30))
 (segment (start 124.351 61.509293) (end 124.351 69.91411) (width 1) (layer "F.Cu") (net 30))
 (segment (start 122.38 59.538293) (end 124.351 61.509293) (width 1) (layer "F.Cu") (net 30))
 (segment (start 124.351 69.91411) (end 122.784817 71.480293) (width 1) (layer "F.Cu") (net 30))
 (segment (start 130 58.668769) (end 130.354 59.02277) (width 1) (layer "F.Cu") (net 27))
 (segment (start 130.354 59.02277) (end 130.354 72.646) (width 1) (layer "F.Cu") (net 27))
 (segment (start 130.354 72.646) (end 123.899707 79.100293) (width 1) (layer "F.Cu") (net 27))
 (segment (start 130 44) (end 130 58.668769) (width 1) (layer "F.Cu") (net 27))
 (segment (start 123.899707 79.100293) (end 122 79.100293) (width 1) (layer "F.Cu") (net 27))
 (segment (start 123.491923 76.560293) (end 122 76.560293) (width 1) (layer "F.Cu") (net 28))
 (segment (start 128.353 59.851611) (end 128.353 71.699216) (width 1) (layer "F.Cu") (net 28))
 (segment (start 128.353 71.699216) (end 123.491923 76.560293) (width 1) (layer "F.Cu") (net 28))
 (segment (start 127.46 58.958611) (end 128.353 59.851611) (width 1) (layer "F.Cu") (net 28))
 (segment (start 127.46 44) (end 127.46 58.958611) (width 1) (layer "F.Cu") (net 28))
 (segment (start 122.784817 84.180293) (end 122 84.180293) (width 1) (layer "F.Cu") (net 26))
 (segment (start 132.54 44) (end 132.54 74.42511) (width 1) (layer "F.Cu") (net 26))
 (segment (start 132.54 74.42511) (end 122.784817 84.180293) (width 1) (layer "F.Cu") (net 26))
 (segment (start 116.326183 41.649) (end 114.949 43.026183) (width 1) (layer "F.Cu") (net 24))
 (segment (start 136.471081 41.649) (end 116.326183 41.649) (width 1) (layer "F.Cu") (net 24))
 (segment (start 121.215183 89.260293) (end 122 89.260293) (width 1) (layer "F.Cu") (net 24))
 (segment (start 137.62 42.797919) (end 136.471081 41.649) (width 1) (layer "F.Cu") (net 24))
 (segment (start 114.949 82.99411) (end 121.215183 89.260293) (width 1) (layer "F.Cu") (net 24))
 (segment (start 137.62 44) (end 137.62 42.797919) (width 1) (layer "F.Cu") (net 24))
 (segment (start 114.949 43.026183) (end 114.949 82.99411) (width 1) (layer "F.Cu") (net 24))
 (segment (start 124.92 44) (end 124.92 59.248451) (width 1) (layer "F.Cu") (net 29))
 (segment (start 126.352 60.680452) (end 126.352 70.870374) (width 1) (layer "F.Cu") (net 29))
 (segment (start 126.352 70.870374) (end 123.202081 74.020293) (width 1) (layer "F.Cu") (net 29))
 (segment (start 123.202081 74.020293) (end 122 74.020293) (width 1) (layer "F.Cu") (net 29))
 (segment (start 124.92 59.248451) (end 126.352 60.680452) (width 1) (layer "F.Cu") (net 29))
 (segment (start 127.75 99.25) (end 127.800293 99.300293) (width 1) (layer "F.Cu") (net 13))
 (segment (start 127.800293 99.300293) (end 139.62 99.300293) (width 1) (layer "F.Cu") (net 13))
 (segment (start 124.646381 115.628571) (end 127.75 112.524952) (width 1) (layer "F.Cu") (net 13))
 (segment (start 124.646381 121.904762) (end 124.646381 115.628571) (width 1) (layer "F.Cu") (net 13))
 (segment (start 127.75 112.524952) (end 127.75 99.25) (width 1) (layer "F.Cu") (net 13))
 (segment (start 132.25 104.380293) (end 132.25 110.51545) (width 1) (layer "F.Cu") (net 11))
 (segment (start 139.62 104.380293) (end 132.25 104.380293) (width 1) (layer "F.Cu") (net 11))
 (segment (start 132.25 110.51545) (end 132.266381 110.531831) (width 1) (layer "F.Cu") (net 11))
 (segment (start 132.266381 110.531831) (end 132.266381 121.904762) (width 1) (layer "F.Cu") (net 11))
 (segment (start 127.186381 115.918413) (end 127.186381 121.904762) (width 1) (layer "F.Cu") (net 12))
 (segment (start 139.62 101.840293) (end 129.910707 101.840293) (width 1) (layer "F.Cu") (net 12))
 (segment (start 129.751 113.353794) (end 127.186381 115.918413) (width 1) (layer "F.Cu") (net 12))
 (segment (start 129.751 102) (end 129.751 113.353794) (width 1) (layer "F.Cu") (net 12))
 (segment (start 129.910707 101.840293) (end 129.751 102) (width 1) (layer "F.Cu") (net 12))
 (segment (start 137.458 109.460293) (end 134.806381 112.111912) (width 1) (layer "F.Cu") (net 10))
 (segment (start 134.806381 112.111912) (end 134.806381 121.904762) (width 1) (layer "F.Cu") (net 10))
 (segment (start 139.62 109.460293) (end 137.458 109.460293) (width 1) (layer "F.Cu") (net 10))
 (segment (start 142.237381 129.455381) (end 142.237381 75.732857) (width 1) (layer "F.Cu") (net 5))
 (segment (start 142.237381 75.732857) (end 140.404817 73.900293) (width 1) (layer "F.Cu") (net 5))
 (segment (start 140.404817 73.900293) (end 139.62 73.900293) (width 1) (layer "F.Cu") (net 5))
 (segment (start 129.726381 126.726381) (end 137.346381 134.346381) (width 1) (layer "F.Cu") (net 5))
 (segment (start 142.7 57.335476) (end 137.269 62.766476) (width 1) (layer "F.Cu") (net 5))
 (segment (start 137.269 62.766476) (end 137.269 73.269) (width 1) (layer "F.Cu") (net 5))
 (segment (start 137.269 73.269) (end 137.900293 73.900293) (width 1) (layer "F.Cu") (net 5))
 (segment (start 142.7 44) (end 142.7 57.335476) (width 1) (layer "F.Cu") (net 5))
 (segment (start 137.346381 134.346381) (end 137.346381 137.992762) (width 1) (layer "F.Cu") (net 5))
 (segment (start 137.346381 134.346381) (end 142.237381 129.455381) (width 1) (layer "F.Cu") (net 5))
 (segment (start 137.900293 73.900293) (end 139.62 73.900293) (width 1) (layer "F.Cu") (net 5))
 (segment (start 129.726381 121.904762) (end 129.726381 126.726381) (width 1) (layer "F.Cu") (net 5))
 (segment (start 137.346381 114.273912) (end 137.346381 121.904762) (width 1) (layer "F.Cu") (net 9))
 (segment (start 139.62 112.000293) (end 137.346381 114.273912) (width 1) (layer "F.Cu") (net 9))
 (segment (start 125.75 97) (end 125.989707 96.760293) (width 1) (layer "F.Cu") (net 14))
 (segment (start 125.75 111.69511) (end 125.75 97) (width 1) (layer "F.Cu") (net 14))
 (segment (start 125.989707 96.760293) (end 139.62 96.760293) (width 1) (layer "F.Cu") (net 14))
 (segment (start 122.106381 115.338729) (end 125.75 111.69511) (width 1) (layer "F.Cu") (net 14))
 (segment (start 122.106381 121.904762) (end 122.106381 115.338729) (width 1) (layer "F.Cu") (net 14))
 (segment (start 62.0265 68.336) (end 62.0265 133.0265) (width 1) (layer "F.Cu") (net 7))
 (segment (start 64.8275 65.535) (end 62.0265 68.336) (width 1) (layer "F.Cu") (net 7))
 (segment (start 64.8275 135.535) (end 123.3907 135.535) (width 1) (layer "F.Cu") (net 7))
 (segment (start 62.0265 133.0265) (end 63.26633 134.26633) (width 1) (layer "F.Cu") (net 7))
 (segment (start 123.3907 135.535) (end 124.646381 136.790681) (width 1) (layer "F.Cu") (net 7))
 (segment (start 124.646381 136.790681) (end 124.646381 137.992762) (width 1) (layer "F.Cu") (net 7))
 (segment (start 63.26633 134.26633) (end 63.412579 134.120081) (width 1) (layer "F.Cu") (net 7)))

